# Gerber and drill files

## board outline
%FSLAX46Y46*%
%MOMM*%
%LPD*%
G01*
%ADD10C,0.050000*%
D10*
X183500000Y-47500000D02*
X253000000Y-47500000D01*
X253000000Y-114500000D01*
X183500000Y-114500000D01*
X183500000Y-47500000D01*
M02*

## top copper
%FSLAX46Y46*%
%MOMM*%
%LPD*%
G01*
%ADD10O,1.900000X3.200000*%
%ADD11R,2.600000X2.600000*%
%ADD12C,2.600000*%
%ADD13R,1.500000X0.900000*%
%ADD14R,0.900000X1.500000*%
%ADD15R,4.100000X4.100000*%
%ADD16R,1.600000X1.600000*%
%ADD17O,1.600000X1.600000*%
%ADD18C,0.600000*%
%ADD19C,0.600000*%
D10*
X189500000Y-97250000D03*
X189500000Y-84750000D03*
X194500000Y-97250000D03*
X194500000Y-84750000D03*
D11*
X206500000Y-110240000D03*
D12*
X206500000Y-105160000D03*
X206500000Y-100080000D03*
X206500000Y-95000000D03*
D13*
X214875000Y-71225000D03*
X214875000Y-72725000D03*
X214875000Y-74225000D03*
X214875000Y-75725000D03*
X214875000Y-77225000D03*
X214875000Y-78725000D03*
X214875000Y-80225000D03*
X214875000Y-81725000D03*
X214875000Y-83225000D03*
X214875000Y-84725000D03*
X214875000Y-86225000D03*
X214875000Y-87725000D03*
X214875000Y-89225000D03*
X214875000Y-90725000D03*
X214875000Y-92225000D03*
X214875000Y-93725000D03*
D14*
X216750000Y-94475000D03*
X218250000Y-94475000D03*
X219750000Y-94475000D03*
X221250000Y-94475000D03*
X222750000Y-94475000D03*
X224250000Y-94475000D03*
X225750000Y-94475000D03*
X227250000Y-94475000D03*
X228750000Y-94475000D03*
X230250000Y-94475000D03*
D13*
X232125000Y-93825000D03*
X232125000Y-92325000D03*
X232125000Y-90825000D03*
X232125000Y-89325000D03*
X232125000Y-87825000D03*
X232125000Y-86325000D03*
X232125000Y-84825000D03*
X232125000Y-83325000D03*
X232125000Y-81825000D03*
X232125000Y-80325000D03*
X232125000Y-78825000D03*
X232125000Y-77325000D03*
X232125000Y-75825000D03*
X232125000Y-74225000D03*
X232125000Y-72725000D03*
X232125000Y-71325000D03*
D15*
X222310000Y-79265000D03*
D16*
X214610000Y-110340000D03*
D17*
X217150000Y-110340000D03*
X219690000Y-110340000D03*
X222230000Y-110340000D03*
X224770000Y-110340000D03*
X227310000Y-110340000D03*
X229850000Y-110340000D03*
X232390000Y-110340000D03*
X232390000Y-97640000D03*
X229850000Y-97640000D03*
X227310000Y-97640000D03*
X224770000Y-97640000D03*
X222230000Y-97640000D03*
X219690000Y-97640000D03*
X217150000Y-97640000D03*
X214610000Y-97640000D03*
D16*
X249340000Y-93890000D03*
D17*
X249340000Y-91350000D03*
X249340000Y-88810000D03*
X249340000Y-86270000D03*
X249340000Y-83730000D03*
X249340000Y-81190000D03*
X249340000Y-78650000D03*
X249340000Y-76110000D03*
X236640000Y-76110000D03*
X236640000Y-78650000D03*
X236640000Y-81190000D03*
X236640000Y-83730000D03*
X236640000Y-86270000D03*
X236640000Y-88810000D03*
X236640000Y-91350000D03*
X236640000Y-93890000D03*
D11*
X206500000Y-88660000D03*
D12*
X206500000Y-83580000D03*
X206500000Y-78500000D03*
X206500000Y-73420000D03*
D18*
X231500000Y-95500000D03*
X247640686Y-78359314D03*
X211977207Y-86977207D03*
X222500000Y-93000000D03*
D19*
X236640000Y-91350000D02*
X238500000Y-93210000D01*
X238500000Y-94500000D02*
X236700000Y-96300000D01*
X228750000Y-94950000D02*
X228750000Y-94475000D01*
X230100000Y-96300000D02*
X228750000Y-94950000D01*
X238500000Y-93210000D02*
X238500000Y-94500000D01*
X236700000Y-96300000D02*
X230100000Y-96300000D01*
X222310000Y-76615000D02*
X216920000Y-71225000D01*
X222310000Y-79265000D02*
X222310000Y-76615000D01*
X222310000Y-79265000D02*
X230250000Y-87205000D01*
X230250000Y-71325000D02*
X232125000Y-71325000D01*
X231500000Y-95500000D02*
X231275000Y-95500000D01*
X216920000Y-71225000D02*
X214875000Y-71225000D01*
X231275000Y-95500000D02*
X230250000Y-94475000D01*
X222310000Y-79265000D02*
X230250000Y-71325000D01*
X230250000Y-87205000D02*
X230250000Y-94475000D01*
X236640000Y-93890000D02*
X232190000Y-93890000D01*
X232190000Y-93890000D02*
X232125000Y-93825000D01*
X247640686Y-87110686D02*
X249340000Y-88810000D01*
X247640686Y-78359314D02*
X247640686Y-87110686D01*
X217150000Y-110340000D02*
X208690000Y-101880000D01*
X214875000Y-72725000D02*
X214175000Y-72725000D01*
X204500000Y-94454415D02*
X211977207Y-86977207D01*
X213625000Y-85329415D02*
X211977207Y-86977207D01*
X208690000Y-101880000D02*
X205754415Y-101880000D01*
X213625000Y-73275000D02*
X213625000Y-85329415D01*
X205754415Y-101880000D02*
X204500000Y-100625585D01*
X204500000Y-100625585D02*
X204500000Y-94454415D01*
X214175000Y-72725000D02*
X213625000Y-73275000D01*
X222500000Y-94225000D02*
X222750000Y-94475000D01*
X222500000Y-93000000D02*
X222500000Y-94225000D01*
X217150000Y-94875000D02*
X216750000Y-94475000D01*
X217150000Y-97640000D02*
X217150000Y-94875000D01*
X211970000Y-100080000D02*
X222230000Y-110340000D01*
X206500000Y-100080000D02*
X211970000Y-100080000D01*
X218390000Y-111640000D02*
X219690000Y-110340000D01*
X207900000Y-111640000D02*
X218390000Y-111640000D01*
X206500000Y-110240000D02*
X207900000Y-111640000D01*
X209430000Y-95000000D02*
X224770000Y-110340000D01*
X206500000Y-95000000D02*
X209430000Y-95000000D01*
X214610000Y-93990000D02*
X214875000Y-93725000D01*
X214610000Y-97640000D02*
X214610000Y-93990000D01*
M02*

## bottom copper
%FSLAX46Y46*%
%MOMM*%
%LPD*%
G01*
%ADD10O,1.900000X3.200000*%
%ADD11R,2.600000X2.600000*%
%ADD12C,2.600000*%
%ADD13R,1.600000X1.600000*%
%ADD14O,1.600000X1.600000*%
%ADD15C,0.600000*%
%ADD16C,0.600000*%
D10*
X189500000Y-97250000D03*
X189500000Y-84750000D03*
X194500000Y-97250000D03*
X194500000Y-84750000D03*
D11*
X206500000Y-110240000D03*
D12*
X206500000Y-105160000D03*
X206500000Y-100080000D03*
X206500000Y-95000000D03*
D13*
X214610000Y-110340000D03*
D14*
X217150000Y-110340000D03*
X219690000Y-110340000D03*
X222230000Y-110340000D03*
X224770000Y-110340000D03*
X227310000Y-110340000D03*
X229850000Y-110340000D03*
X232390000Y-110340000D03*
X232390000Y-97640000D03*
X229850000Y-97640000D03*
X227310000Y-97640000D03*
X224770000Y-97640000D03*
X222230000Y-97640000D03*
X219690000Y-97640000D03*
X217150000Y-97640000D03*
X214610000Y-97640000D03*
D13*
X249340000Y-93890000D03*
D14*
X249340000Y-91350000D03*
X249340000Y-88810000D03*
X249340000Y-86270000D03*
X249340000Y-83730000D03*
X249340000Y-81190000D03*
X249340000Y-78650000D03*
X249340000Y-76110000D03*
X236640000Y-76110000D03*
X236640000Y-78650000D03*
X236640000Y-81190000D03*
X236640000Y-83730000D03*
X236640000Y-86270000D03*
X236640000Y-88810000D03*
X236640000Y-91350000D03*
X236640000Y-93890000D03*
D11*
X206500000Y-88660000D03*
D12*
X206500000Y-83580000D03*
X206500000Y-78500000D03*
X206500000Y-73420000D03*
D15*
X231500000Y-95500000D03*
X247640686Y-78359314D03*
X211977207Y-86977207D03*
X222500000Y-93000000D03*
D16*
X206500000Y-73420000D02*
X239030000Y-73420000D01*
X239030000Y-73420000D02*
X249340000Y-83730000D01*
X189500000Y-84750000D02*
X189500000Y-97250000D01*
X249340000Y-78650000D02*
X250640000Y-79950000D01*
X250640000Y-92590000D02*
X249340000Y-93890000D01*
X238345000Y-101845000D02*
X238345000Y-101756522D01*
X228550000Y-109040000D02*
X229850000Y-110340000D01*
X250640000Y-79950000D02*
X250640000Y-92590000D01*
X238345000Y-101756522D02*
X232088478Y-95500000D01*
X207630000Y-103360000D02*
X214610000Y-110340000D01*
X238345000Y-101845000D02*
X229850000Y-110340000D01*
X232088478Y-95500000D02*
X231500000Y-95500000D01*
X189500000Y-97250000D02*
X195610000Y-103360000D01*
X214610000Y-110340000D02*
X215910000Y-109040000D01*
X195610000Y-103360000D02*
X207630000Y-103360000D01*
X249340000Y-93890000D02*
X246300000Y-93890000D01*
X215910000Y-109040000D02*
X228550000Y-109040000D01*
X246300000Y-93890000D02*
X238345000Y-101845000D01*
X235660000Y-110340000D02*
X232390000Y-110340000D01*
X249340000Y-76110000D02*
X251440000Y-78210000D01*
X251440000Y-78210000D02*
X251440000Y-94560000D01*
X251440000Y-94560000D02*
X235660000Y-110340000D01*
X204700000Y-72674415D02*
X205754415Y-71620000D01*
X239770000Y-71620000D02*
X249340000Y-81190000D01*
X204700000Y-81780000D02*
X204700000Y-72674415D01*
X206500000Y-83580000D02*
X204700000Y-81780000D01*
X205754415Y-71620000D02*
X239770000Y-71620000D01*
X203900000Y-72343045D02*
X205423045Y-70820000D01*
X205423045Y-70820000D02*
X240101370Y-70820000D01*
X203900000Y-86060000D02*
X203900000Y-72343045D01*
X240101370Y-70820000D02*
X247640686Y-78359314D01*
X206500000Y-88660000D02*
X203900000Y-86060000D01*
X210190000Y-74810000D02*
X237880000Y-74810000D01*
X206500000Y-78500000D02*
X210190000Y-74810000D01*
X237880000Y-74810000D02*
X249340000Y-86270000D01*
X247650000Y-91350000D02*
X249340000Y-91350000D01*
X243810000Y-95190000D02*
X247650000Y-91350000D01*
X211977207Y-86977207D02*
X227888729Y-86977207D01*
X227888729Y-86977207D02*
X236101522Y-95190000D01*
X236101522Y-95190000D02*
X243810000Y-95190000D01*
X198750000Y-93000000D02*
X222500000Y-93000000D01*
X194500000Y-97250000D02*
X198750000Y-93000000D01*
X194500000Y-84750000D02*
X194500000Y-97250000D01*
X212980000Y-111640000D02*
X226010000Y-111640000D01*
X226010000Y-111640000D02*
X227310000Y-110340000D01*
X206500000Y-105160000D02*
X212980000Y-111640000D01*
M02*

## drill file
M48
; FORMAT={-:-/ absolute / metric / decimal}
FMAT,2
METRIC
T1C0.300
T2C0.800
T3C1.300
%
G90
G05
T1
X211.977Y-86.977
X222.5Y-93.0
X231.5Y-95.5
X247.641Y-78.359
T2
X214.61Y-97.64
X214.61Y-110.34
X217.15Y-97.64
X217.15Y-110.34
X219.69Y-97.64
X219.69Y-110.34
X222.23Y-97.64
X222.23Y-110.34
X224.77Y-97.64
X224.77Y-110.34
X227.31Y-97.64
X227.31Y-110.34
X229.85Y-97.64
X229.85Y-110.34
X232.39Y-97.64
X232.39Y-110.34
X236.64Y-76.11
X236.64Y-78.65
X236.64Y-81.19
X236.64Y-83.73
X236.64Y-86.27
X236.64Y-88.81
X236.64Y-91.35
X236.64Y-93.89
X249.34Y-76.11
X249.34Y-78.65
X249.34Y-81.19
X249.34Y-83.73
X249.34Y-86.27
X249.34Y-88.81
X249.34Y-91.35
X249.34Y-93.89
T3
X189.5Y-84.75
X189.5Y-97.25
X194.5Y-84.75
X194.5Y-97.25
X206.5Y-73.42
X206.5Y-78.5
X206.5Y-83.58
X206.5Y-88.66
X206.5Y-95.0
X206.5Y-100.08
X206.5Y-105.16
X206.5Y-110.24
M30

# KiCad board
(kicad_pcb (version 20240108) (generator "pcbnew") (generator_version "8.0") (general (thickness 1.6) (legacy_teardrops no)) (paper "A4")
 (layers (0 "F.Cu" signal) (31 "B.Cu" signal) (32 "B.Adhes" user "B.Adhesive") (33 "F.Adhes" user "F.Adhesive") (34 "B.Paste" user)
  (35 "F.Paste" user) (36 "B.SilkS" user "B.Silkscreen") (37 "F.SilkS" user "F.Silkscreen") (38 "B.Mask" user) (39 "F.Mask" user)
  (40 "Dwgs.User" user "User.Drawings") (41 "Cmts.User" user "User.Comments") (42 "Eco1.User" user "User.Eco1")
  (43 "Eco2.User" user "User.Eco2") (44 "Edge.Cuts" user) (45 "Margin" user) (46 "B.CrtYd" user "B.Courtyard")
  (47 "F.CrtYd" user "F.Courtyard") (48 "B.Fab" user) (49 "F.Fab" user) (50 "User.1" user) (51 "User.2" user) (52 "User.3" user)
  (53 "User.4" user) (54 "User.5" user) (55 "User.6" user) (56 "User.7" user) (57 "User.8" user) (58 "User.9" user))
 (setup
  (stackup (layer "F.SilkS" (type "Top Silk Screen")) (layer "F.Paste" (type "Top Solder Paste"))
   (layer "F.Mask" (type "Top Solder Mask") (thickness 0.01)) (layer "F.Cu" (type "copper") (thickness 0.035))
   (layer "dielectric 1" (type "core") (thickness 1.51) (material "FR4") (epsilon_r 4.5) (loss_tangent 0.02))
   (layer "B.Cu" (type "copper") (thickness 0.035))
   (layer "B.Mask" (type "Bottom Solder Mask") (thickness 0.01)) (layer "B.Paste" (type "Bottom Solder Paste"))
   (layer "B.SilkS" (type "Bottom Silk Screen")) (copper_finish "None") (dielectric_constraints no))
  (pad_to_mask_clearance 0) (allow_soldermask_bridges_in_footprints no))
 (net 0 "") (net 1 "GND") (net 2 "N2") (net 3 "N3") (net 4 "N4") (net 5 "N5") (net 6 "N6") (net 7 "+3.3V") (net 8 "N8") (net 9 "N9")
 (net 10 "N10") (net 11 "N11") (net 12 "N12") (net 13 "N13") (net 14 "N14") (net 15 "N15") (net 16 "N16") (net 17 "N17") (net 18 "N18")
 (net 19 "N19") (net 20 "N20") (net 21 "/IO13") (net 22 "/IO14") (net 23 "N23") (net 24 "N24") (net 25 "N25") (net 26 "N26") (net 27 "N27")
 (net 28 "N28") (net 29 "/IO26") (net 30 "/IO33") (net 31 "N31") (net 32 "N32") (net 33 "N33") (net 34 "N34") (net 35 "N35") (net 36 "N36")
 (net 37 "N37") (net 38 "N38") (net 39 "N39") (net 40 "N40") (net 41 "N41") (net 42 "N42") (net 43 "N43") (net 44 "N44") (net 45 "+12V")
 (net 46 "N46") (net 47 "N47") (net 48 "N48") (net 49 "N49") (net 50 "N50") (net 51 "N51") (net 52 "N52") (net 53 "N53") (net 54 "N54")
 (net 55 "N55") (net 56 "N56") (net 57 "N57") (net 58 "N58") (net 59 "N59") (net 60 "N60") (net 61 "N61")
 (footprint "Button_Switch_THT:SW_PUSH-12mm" (layer "F.Cu") (at 189.5 97.25 90)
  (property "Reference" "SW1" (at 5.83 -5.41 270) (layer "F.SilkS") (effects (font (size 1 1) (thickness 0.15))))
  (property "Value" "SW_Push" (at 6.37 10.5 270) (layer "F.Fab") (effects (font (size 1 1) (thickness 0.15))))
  (pad "1" thru_hole oval (at 0 0 90) (size 3.2 1.9) (drill 1.3) (layers "*.Cu" "*.Mask") (remove_unused_layers no) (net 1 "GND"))
  (pad "1" thru_hole oval (at 12.5 0 90) (size 3.2 1.9) (drill 1.3) (layers "*.Cu" "*.Mask") (remove_unused_layers no) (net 1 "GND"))
  (pad "2" thru_hole oval (at 0 5 90) (size 3.2 1.9) (drill 1.3) (layers "*.Cu" "*.Mask") (remove_unused_layers no) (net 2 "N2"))
  (pad "2" thru_hole oval (at 12.5 5 90) (size 3.2 1.9) (drill 1.3) (layers "*.Cu" "*.Mask") (remove_unused_layers no) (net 2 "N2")))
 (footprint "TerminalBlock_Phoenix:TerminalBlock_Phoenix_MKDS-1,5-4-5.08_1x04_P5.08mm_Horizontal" (layer "F.Cu") (at 206.5 110.24 90)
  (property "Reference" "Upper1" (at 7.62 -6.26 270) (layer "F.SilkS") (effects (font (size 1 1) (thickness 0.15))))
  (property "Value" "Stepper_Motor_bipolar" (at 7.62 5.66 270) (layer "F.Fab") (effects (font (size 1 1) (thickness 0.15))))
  (pad "1" thru_hole rect (at 0 0 90) (size 2.6 2.6) (drill 1.3) (layers "*.Cu" "*.Mask") (remove_unused_layers no) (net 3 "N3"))
  (pad "2" thru_hole circle (at 5.08 0 90) (size 2.6 2.6) (drill 1.3) (layers "*.Cu" "*.Mask") (remove_unused_layers no) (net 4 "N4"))
  (pad "3" thru_hole circle (at 10.16 0 90) (size 2.6 2.6) (drill 1.3) (layers "*.Cu" "*.Mask") (remove_unused_layers no) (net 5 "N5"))
  (pad "4" thru_hole circle (at 15.24 0 90) (size 2.6 2.6) (drill 1.3) (layers "*.Cu" "*.Mask") (remove_unused_layers no) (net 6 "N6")))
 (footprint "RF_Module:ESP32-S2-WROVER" (layer "F.Cu") (at 223.5 83)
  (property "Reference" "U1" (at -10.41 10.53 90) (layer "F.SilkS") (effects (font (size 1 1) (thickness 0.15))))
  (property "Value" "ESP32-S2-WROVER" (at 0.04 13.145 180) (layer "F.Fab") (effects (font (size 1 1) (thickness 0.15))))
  (pad "1" smd rect (at -8.625 -11.775) (size 1.5 0.9) (layers "F.Cu" "F.Paste" "F.Mask") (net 1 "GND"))
  (pad "2" smd rect (at -8.625 -10.275) (size 1.5 0.9) (layers "F.Cu" "F.Paste" "F.Mask") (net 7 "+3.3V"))
  (pad "3" smd rect (at -8.625 -8.775) (size 1.5 0.9) (layers "F.Cu" "F.Paste" "F.Mask") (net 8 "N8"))
  (pad "4" smd rect (at -8.625 -7.275) (size 1.5 0.9) (layers "F.Cu" "F.Paste" "F.Mask") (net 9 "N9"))
  (pad "5" smd rect (at -8.625 -5.775) (size 1.5 0.9) (layers "F.Cu" "F.Paste" "F.Mask") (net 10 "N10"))
  (pad "6" smd rect (at -8.625 -4.275) (size 1.5 0.9) (layers "F.Cu" "F.Paste" "F.Mask") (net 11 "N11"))
  (pad "7" smd rect (at -8.625 -2.775) (size 1.5 0.9) (layers "F.Cu" "F.Paste" "F.Mask") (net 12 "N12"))
  (pad "8" smd rect (at -8.625 -1.275) (size 1.5 0.9) (layers "F.Cu" "F.Paste" "F.Mask") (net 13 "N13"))
  (pad "9" smd rect (at -8.625 0.225) (size 1.5 0.9) (layers "F.Cu" "F.Paste" "F.Mask") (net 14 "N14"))
  (pad "10" smd rect (at -8.625 1.725) (size 1.5 0.9) (layers "F.Cu" "F.Paste" "F.Mask") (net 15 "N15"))
  (pad "11" smd rect (at -8.625 3.225) (size 1.5 0.9) (layers "F.Cu" "F.Paste" "F.Mask") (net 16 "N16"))
  (pad "12" smd rect (at -8.625 4.725) (size 1.5 0.9) (layers "F.Cu" "F.Paste" "F.Mask") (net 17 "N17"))
  (pad "13" smd rect (at -8.625 6.225) (size 1.5 0.9) (layers "F.Cu" "F.Paste" "F.Mask") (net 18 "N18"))
  (pad "14" smd rect (at -8.625 7.725) (size 1.5 0.9) (layers "F.Cu" "F.Paste" "F.Mask") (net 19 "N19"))
  (pad "15" smd rect (at -8.625 9.225 180) (size 1.5 0.9) (layers "F.Cu" "F.Paste" "F.Mask") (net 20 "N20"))
  (pad "16" smd rect (at -8.625 10.725 180) (size 1.5 0.9) (layers "F.Cu" "F.Paste" "F.Mask") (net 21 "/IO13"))
  (pad "17" smd rect (at -6.75 11.475) (size 0.9 1.5) (layers "F.Cu" "F.Paste" "F.Mask") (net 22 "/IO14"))
  (pad "18" smd rect (at -5.25 11.475) (size 0.9 1.5) (layers "F.Cu" "F.Paste" "F.Mask") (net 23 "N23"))
  (pad "19" smd rect (at -3.75 11.475) (size 0.9 1.5) (layers "F.Cu" "F.Paste" "F.Mask") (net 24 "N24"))
  (pad "20" smd rect (at -2.25 11.475) (size 0.9 1.5) (layers "F.Cu" "F.Paste" "F.Mask") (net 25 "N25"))
  (pad "21" smd rect (at -0.75 11.475) (size 0.9 1.5) (layers "F.Cu" "F.Paste" "F.Mask") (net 2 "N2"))
  (pad "22" smd rect (at 0.75 11.475) (size 0.9 1.5) (layers "F.Cu" "F.Paste" "F.Mask") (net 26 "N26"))
  (pad "23" smd rect (at 2.25 11.475) (size 0.9 1.5) (layers "F.Cu" "F.Paste" "F.Mask") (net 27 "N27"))
  (pad "24" smd rect (at 3.75 11.475) (size 0.9 1.5) (layers "F.Cu" "F.Paste" "F.Mask") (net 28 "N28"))
  (pad "25" smd rect (at 5.25 11.475) (size 0.9 1.5) (layers "F.Cu" "F.Paste" "F.Mask") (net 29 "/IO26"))
  (pad "26" smd rect (at 6.75 11.475) (size 0.9 1.5) (layers "F.Cu" "F.Paste" "F.Mask") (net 1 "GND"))
  (pad "27" smd rect (at 8.625 10.825) (size 1.5 0.9) (layers "F.Cu" "F.Paste" "F.Mask") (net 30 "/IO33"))
  (pad "28" smd rect (at 8.625 9.325) (size 1.5 0.9) (layers "F.Cu" "F.Paste" "F.Mask") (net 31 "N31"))
  (pad "29" smd rect (at 8.625 7.825) (size 1.5 0.9) (layers "F.Cu" "F.Paste" "F.Mask") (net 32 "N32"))
  (pad "30" smd rect (at 8.625 6.325) (size 1.5 0.9) (layers "F.Cu" "F.Paste" "F.Mask") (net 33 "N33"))
  (pad "31" smd rect (at 8.625 4.825) (size 1.5 0.9) (layers "F.Cu" "F.Paste" "F.Mask") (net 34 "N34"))
  (pad "32" smd rect (at 8.625 3.325) (size 1.5 0.9) (layers "F.Cu" "F.Paste" "F.Mask") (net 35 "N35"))
  (pad "33" smd rect (at 8.625 1.825) (size 1.5 0.9) (layers "F.Cu" "F.Paste" "F.Mask") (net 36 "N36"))
  (pad "34" smd rect (at 8.625 0.325) (size 1.5 0.9) (layers "F.Cu" "F.Paste" "F.Mask") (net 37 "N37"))
  (pad "35" smd rect (at 8.625 -1.175) (size 1.5 0.9) (layers "F.Cu" "F.Paste" "F.Mask") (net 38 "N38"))
  (pad "36" smd rect (at 8.625 -2.675) (size 1.5 0.9) (layers "F.Cu" "F.Paste" "F.Mask") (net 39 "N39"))
  (pad "37" smd rect (at 8.625 -4.175) (size 1.5 0.9) (layers "F.Cu" "F.Paste" "F.Mask") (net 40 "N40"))
  (pad "38" smd rect (at 8.625 -5.675) (size 1.5 0.9) (layers "F.Cu" "F.Paste" "F.Mask") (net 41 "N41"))
  (pad "39" smd rect (at 8.625 -7.175) (size 1.5 0.9) (layers "F.Cu" "F.Paste" "F.Mask") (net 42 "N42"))
  (pad "40" smd rect (at 8.625 -8.775) (size 1.5 0.9) (layers "F.Cu" "F.Paste" "F.Mask") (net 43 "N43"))
  (pad "41" smd rect (at 8.625 -10.275) (size 1.5 0.9) (layers "F.Cu" "F.Paste" "F.Mask") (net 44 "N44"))
  (pad "42" smd rect (at 8.625 -11.675) (size 1.5 0.9) (layers "F.Cu" "F.Paste" "F.Mask") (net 1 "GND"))
  (pad "43" smd rect (at -1.19 -3.735) (size 4.1 4.1) (layers "F.Cu" "F.Paste" "F.Mask") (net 1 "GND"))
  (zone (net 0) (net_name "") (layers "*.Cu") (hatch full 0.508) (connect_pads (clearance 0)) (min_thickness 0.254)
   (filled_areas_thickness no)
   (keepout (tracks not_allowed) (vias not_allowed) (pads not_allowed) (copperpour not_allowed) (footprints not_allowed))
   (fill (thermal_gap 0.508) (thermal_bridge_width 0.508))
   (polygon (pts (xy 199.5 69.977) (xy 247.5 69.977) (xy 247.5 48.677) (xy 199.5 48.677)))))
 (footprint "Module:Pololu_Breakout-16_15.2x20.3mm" (layer "F.Cu") (at 214.61 110.34 90)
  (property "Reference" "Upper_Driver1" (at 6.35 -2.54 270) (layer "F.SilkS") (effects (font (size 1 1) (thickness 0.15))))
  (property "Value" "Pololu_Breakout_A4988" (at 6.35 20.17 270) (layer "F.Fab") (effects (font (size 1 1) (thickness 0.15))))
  (pad "1" thru_hole rect (at 0 0 90) (size 1.6 1.6) (drill 0.8) (layers "*.Cu" "*.Mask") (remove_unused_layers no) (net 1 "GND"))
  (pad "2" thru_hole oval (at 0 2.54 90) (size 1.6 1.6) (drill 0.8) (layers "*.Cu" "*.Mask") (remove_unused_layers no) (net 7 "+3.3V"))
  (pad "3" thru_hole oval (at 0 5.08 90) (size 1.6 1.6) (drill 0.8) (layers "*.Cu" "*.Mask") (remove_unused_layers no) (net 3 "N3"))
  (pad "4" thru_hole oval (at 0 7.62 90) (size 1.6 1.6) (drill 0.8) (layers "*.Cu" "*.Mask") (remove_unused_layers no) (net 5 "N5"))
  (pad "5" thru_hole oval (at 0 10.16 90) (size 1.6 1.6) (drill 0.8) (layers "*.Cu" "*.Mask") (remove_unused_layers no) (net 6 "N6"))
  (pad "6" thru_hole oval (at 0 12.7 90) (size 1.6 1.6) (drill 0.8) (layers "*.Cu" "*.Mask") (remove_unused_layers no) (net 4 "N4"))
  (pad "7" thru_hole oval (at 0 15.24 90) (size 1.6 1.6) (drill 0.8) (layers "*.Cu" "*.Mask") (remove_unused_layers no) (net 1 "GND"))
  (pad "8" thru_hole oval (at 0 17.78 90) (size 1.6 1.6) (drill 0.8) (layers "*.Cu" "*.Mask") (remove_unused_layers no) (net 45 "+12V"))
  (pad "9" thru_hole oval (at 12.7 17.78 90) (size 1.6 1.6) (drill 0.8) (layers "*.Cu" "*.Mask") (remove_unused_layers no) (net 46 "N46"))
  (pad "10" thru_hole oval (at 12.7 15.24 90) (size 1.6 1.6) (drill 0.8) (layers "*.Cu" "*.Mask") (remove_unused_layers no) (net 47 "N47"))
  (pad "11" thru_hole oval (at 12.7 12.7 90) (size 1.6 1.6) (drill 0.8) (layers "*.Cu" "*.Mask") (remove_unused_layers no) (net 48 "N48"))
  (pad "12" thru_hole oval (at 12.7 10.16 90) (size 1.6 1.6) (drill 0.8) (layers "*.Cu" "*.Mask") (remove_unused_layers no) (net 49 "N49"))
  (pad "13" thru_hole oval (at 12.7 7.62 90) (size 1.6 1.6) (drill 0.8) (layers "*.Cu" "*.Mask") (remove_unused_layers no) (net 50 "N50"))
  (pad "14" thru_hole oval (at 12.7 5.08 90) (size 1.6 1.6) (drill 0.8) (layers "*.Cu" "*.Mask") (remove_unused_layers no) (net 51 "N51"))
  (pad "15" thru_hole oval (at 12.7 2.54 90) (size 1.6 1.6) (drill 0.8) (layers "*.Cu" "*.Mask") (remove_unused_layers no) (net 22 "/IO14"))
  (pad "16" thru_hole oval (at 12.7 0 90) (size 1.6 1.6) (drill 0.8) (layers "*.Cu" "*.Mask") (remove_unused_layers no) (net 21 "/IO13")))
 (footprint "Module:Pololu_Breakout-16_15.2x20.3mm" (layer "F.Cu") (at 249.34 93.89 180)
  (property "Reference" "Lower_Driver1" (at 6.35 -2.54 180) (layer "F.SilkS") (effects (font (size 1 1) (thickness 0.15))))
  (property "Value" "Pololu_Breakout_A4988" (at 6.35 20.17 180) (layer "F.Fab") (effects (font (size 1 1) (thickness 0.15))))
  (pad "1" thru_hole rect (at 0 0 180) (size 1.6 1.6) (drill 0.8) (layers "*.Cu" "*.Mask") (remove_unused_layers no) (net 1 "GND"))
  (pad "2" thru_hole oval (at 0 2.54 180) (size 1.6 1.6) (drill 0.8) (layers "*.Cu" "*.Mask") (remove_unused_layers no) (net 7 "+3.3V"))
  (pad "3" thru_hole oval (at 0 5.08 180) (size 1.6 1.6) (drill 0.8) (layers "*.Cu" "*.Mask") (remove_unused_layers no) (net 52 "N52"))
  (pad "4" thru_hole oval (at 0 7.62 180) (size 1.6 1.6) (drill 0.8) (layers "*.Cu" "*.Mask") (remove_unused_layers no) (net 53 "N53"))
  (pad "5" thru_hole oval (at 0 10.16 180) (size 1.6 1.6) (drill 0.8) (layers "*.Cu" "*.Mask") (remove_unused_layers no) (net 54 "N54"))
  (pad "6" thru_hole oval (at 0 12.7 180) (size 1.6 1.6) (drill 0.8) (layers "*.Cu" "*.Mask") (remove_unused_layers no) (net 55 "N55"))
  (pad "7" thru_hole oval (at 0 15.24 180) (size 1.6 1.6) (drill 0.8) (layers "*.Cu" "*.Mask") (remove_unused_layers no) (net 1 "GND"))
  (pad "8" thru_hole oval (at 0 17.78 180) (size 1.6 1.6) (drill 0.8) (layers "*.Cu" "*.Mask") (remove_unused_layers no) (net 45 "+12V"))
  (pad "9" thru_hole oval (at 12.7 17.78 180) (size 1.6 1.6) (drill 0.8) (layers "*.Cu" "*.Mask") (remove_unused_layers no) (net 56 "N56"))
  (pad "10" thru_hole oval (at 12.7 15.24 180) (size 1.6 1.6) (drill 0.8) (layers "*.Cu" "*.Mask") (remove_unused_layers no) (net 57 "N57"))
  (pad "11" thru_hole oval (at 12.7 12.7 180) (size 1.6 1.6) (drill 0.8) (layers "*.Cu" "*.Mask") (remove_unused_layers no) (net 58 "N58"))
  (pad "12" thru_hole oval (at 12.7 10.16 180) (size 1.6 1.6) (drill 0.8) (layers "*.Cu" "*.Mask") (remove_unused_layers no) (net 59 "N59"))
  (pad "13" thru_hole oval (at 12.7 7.62 180) (size 1.6 1.6) (drill 0.8) (layers "*.Cu" "*.Mask") (remove_unused_layers no) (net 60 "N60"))
  (pad "14" thru_hole oval (at 12.7 5.08 180) (size 1.6 1.6) (drill 0.8) (layers "*.Cu" "*.Mask") (remove_unused_layers no) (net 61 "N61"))
  (pad "15" thru_hole oval (at 12.7 2.54 180) (size 1.6 1.6) (drill 0.8) (layers "*.Cu" "*.Mask") (remove_unused_layers no) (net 29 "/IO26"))
  (pad "16" thru_hole oval (at 12.7 0 180) (size 1.6 1.6) (drill 0.8) (layers "*.Cu" "*.Mask") (remove_unused_layers no) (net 30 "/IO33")))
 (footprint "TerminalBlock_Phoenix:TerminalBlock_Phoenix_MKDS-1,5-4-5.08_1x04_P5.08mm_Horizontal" (layer "F.Cu") (at 206.5 88.66 90)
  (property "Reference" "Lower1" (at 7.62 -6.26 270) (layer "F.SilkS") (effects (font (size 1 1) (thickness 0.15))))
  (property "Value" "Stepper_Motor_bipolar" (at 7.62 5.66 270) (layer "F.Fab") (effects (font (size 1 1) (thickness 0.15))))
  (pad "1" thru_hole rect (at 0 0 90) (size 2.6 2.6) (drill 1.3) (layers "*.Cu" "*.Mask") (remove_unused_layers no) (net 52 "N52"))
  (pad "2" thru_hole circle (at 5.08 0 90) (size 2.6 2.6) (drill 1.3) (layers "*.Cu" "*.Mask") (remove_unused_layers no) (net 55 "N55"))
  (pad "3" thru_hole circle (at 10.16 0 90) (size 2.6 2.6) (drill 1.3) (layers "*.Cu" "*.Mask") (remove_unused_layers no) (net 53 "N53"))
  (pad "4" thru_hole circle (at 15.24 0 90) (size 2.6 2.6) (drill 1.3) (layers "*.Cu" "*.Mask") (remove_unused_layers no) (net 54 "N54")))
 (gr_rect (start 183.5 47.5) (end 253 114.5) (stroke (width 0.05) (type default)) (fill none) (layer "Edge.Cuts"))
 (segment (start 206.5 73.42) (end 239.03 73.42) (width 0.6) (layer "B.Cu") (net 54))
 (segment (start 239.03 73.42) (end 249.34 83.73) (width 0.6) (layer "B.Cu") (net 54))
 (segment (start 236.64 91.35) (end 238.5 93.21) (width 0.6) (layer "F.Cu") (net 29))
 (segment (start 238.5 94.5) (end 236.7 96.3) (width 0.6) (layer "F.Cu") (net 29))
 (segment (start 228.75 94.95) (end 228.75 94.475) (width 0.6) (layer "F.Cu") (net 29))
 (segment (start 230.1 96.3) (end 228.75 94.95) (width 0.6) (layer "F.Cu") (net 29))
 (segment (start 238.5 93.21) (end 238.5 94.5) (width 0.6) (layer "F.Cu") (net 29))
 (segment (start 236.7 96.3) (end 230.1 96.3) (width 0.6) (layer "F.Cu") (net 29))
 (segment (start 222.31 76.615) (end 216.92 71.225) (width 0.6) (layer "F.Cu") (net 1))
 (segment (start 222.31 79.265) (end 222.31 76.615) (width 0.6) (layer "F.Cu") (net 1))
 (segment (start 222.31 79.265) (end 230.25 87.205) (width 0.6) (layer "F.Cu") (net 1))
 (segment (start 230.25 71.325) (end 232.125 71.325) (width 0.6) (layer "F.Cu") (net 1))
 (segment (start 231.5 95.5) (end 231.275 95.5) (width 0.6) (layer "F.Cu") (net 1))
 (segment (start 216.92 71.225) (end 214.875 71.225) (width 0.6) (layer "F.Cu") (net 1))
 (segment (start 231.275 95.5) (end 230.25 94.475) (width 0.6) (layer "F.Cu") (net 1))
 (segment (start 222.31 79.265) (end 230.25 71.325) (width 0.6) (layer "F.Cu") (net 1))
 (segment (start 230.25 87.205) (end 230.25 94.475) (width 0.6) (layer "F.Cu") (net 1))
 (via (at 231.5 95.5) (size 0.6) (drill 0.3) (layers "F.Cu" "B.Cu") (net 1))
 (segment (start 189.5 84.75) (end 189.5 97.25) (width 0.6) (layer "B.Cu") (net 1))
 (segment (start 249.34 78.65) (end 250.64 79.95) (width 0.6) (layer "B.Cu") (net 1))
 (segment (start 250.64 92.59) (end 249.34 93.89) (width 0.6) (layer "B.Cu") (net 1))
 (segment (start 238.345 101.845) (end 238.345 101.756522) (width 0.6) (layer "B.Cu") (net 1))
 (segment (start 228.55 109.04) (end 229.85 110.34) (width 0.6) (layer "B.Cu") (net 1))
 (segment (start 250.64 79.95) (end 250.64 92.59) (width 0.6) (layer "B.Cu") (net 1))
 (segment (start 238.345 101.756522) (end 232.088478 95.5) (width 0.6) (layer "B.Cu") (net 1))
 (segment (start 207.63 103.36) (end 214.61 110.34) (width 0.6) (layer "B.Cu") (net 1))
 (segment (start 238.345 101.845) (end 229.85 110.34) (width 0.6) (layer "B.Cu") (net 1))
 (segment (start 232.088478 95.5) (end 231.5 95.5) (width 0.6) (layer "B.Cu") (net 1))
 (segment (start 189.5 97.25) (end 195.61 103.36) (width 0.6) (layer "B.Cu") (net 1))
 (segment (start 214.61 110.34) (end 215.91 109.04) (width 0.6) (layer "B.Cu") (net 1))
 (segment (start 195.61 103.36) (end 207.63 103.36) (width 0.6) (layer "B.Cu") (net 1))
 (segment (start 249.34 93.89) (end 246.3 93.89) (width 0.6) (layer "B.Cu") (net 1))
 (segment (start 215.91 109.04) (end 228.55 109.04) (width 0.6) (layer "B.Cu") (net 1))
 (segment (start 246.3 93.89) (end 238.345 101.845) (width 0.6) (layer "B.Cu") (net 1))
 (segment (start 235.66 110.34) (end 232.39 110.34) (width 0.6) (layer "B.Cu") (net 45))
 (segment (start 249.34 76.11) (end 251.44 78.21) (width 0.6) (layer "B.Cu") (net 45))
 (segment (start 251.44 78.21) (end 251.44 94.56) (width 0.6) (layer "B.Cu") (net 45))
 (segment (start 251.44 94.56) (end 235.66 110.34) (width 0.6) (layer "B.Cu") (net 45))
 (segment (start 204.7 72.674415) (end 205.754415 71.62) (width 0.6) (layer "B.Cu") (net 55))
 (segment (start 239.77 71.62) (end 249.34 81.19) (width 0.6) (layer "B.Cu") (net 55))
 (segment (start 204.7 81.78) (end 204.7 72.674415) (width 0.6) (layer "B.Cu") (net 55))
 (segment (start 206.5 83.58) (end 204.7 81.78) (width 0.6) (layer "B.Cu") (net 55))
 (segment (start 205.754415 71.62) (end 239.77 71.62) (width 0.6) (layer "B.Cu") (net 55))
 (segment (start 236.64 93.89) (end 232.19 93.89) (width 0.6) (layer "F.Cu") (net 30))
 (segment (start 232.19 93.89) (end 232.125 93.825) (width 0.6) (layer "F.Cu") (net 30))
 (segment (start 247.640686 87.110686) (end 249.34 88.81) (width 0.6) (layer "F.Cu") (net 52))
 (segment (start 247.640686 78.359314) (end 247.640686 87.110686) (width 0.6) (layer "F.Cu") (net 52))
 (via (at 247.640686 78.359314) (size 0.6) (drill 0.3) (layers "F.Cu" "B.Cu") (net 52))
 (segment (start 203.9 72.343045) (end 205.423045 70.82) (width 0.6) (layer "B.Cu") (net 52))
 (segment (start 205.423045 70.82) (end 240.10137 70.82) (width 0.6) (layer "B.Cu") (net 52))
 (segment (start 203.9 86.06) (end 203.9 72.343045) (width 0.6) (layer "B.Cu") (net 52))
 (segment (start 240.10137 70.82) (end 247.640686 78.359314) (width 0.6) (layer "B.Cu") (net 52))
 (segment (start 206.5 88.66) (end 203.9 86.06) (width 0.6) (layer "B.Cu") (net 52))
 (segment (start 210.19 74.81) (end 237.88 74.81) (width 0.6) (layer "B.Cu") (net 53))
 (segment (start 206.5 78.5) (end 210.19 74.81) (width 0.6) (layer "B.Cu") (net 53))
 (segment (start 237.88 74.81) (end 249.34 86.27) (width 0.6) (layer "B.Cu") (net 53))
 (segment (start 217.15 110.34) (end 208.69 101.88) (width 0.6) (layer "F.Cu") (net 7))
 (segment (start 214.875 72.725) (end 214.175 72.725) (width 0.6) (layer "F.Cu") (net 7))
 (segment (start 204.5 94.454415) (end 211.977207 86.977207) (width 0.6) (layer "F.Cu") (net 7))
 (segment (start 213.625 85.329415) (end 211.977207 86.977207) (width 0.6) (layer "F.Cu") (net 7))
 (segment (start 208.69 101.88) (end 205.754415 101.88) (width 0.6) (layer "F.Cu") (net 7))
 (segment (start 213.625 73.275) (end 213.625 85.329415) (width 0.6) (layer "F.Cu") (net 7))
 (segment (start 205.754415 101.88) (end 204.5 100.625585) (width 0.6) (layer "F.Cu") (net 7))
 (segment (start 204.5 100.625585) (end 204.5 94.454415) (width 0.6) (layer "F.Cu") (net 7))
 (segment (start 214.175 72.725) (end 213.625 73.275) (width 0.6) (layer "F.Cu") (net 7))
 (via (at 211.977207 86.977207) (size 0.6) (drill 0.3) (layers "F.Cu" "B.Cu") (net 7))
 (segment (start 247.65 91.35) (end 249.34 91.35) (width 0.6) (layer "B.Cu") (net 7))
 (segment (start 243.81 95.19) (end 247.65 91.35) (width 0.6) (layer "B.Cu") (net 7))
 (segment (start 211.977207 86.977207) (end 227.888729 86.977207) (width 0.6) (layer "B.Cu") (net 7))
 (segment (start 227.888729 86.977207) (end 236.101522 95.19) (width 0.6) (layer "B.Cu") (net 7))
 (segment (start 236.101522 95.19) (end 243.81 95.19) (width 0.6) (layer "B.Cu") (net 7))
 (segment (start 222.5 94.225) (end 222.75 94.475) (width 0.6) (layer "F.Cu") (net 2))
 (segment (start 222.5 93) (end 222.5 94.225) (width 0.6) (layer "F.Cu") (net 2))
 (via (at 222.5 93) (size 0.6) (drill 0.3) (layers "F.Cu" "B.Cu") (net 2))
 (segment (start 198.75 93) (end 222.5 93) (width 0.6) (layer "B.Cu") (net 2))
 (segment (start 194.5 97.25) (end 198.75 93) (width 0.6) (layer "B.Cu") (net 2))
 (segment (start 194.5 84.75) (end 194.5 97.25) (width 0.6) (layer "B.Cu") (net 2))
 (segment (start 217.15 94.875) (end 216.75 94.475) (width 0.6) (layer "F.Cu") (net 22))
 (segment (start 217.15 97.64) (end 217.15 94.875) (width 0.6) (layer "F.Cu") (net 22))
 (segment (start 211.97 100.08) (end 222.23 110.34) (width 0.6) (layer "F.Cu") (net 5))
 (segment (start 206.5 100.08) (end 211.97 100.08) (width 0.6) (layer "F.Cu") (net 5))
 (segment (start 218.39 111.64) (end 219.69 110.34) (width 0.6) (layer "F.Cu") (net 3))
 (segment (start 207.9 111.64) (end 218.39 111.64) (width 0.6) (layer "F.Cu") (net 3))
 (segment (start 206.5 110.24) (end 207.9 111.64) (width 0.6) (layer "F.Cu") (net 3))
 (segment (start 209.43 95) (end 224.77 110.34) (width 0.6) (layer "F.Cu") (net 6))
 (segment (start 206.5 95) (end 209.43 95) (width 0.6) (layer "F.Cu") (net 6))
 (segment (start 212.98 111.64) (end 226.01 111.64) (width 0.6) (layer "B.Cu") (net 4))
 (segment (start 226.01 111.64) (end 227.31 110.34) (width 0.6) (layer "B.Cu") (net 4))
 (segment (start 206.5 105.16) (end 212.98 111.64) (width 0.6) (layer "B.Cu") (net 4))
 (segment (start 214.61 93.99) (end 214.875 93.725) (width 0.6) (layer "F.Cu") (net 21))
 (segment (start 214.61 97.64) (end 214.61 93.99) (width 0.6) (layer "F.Cu") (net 21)))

